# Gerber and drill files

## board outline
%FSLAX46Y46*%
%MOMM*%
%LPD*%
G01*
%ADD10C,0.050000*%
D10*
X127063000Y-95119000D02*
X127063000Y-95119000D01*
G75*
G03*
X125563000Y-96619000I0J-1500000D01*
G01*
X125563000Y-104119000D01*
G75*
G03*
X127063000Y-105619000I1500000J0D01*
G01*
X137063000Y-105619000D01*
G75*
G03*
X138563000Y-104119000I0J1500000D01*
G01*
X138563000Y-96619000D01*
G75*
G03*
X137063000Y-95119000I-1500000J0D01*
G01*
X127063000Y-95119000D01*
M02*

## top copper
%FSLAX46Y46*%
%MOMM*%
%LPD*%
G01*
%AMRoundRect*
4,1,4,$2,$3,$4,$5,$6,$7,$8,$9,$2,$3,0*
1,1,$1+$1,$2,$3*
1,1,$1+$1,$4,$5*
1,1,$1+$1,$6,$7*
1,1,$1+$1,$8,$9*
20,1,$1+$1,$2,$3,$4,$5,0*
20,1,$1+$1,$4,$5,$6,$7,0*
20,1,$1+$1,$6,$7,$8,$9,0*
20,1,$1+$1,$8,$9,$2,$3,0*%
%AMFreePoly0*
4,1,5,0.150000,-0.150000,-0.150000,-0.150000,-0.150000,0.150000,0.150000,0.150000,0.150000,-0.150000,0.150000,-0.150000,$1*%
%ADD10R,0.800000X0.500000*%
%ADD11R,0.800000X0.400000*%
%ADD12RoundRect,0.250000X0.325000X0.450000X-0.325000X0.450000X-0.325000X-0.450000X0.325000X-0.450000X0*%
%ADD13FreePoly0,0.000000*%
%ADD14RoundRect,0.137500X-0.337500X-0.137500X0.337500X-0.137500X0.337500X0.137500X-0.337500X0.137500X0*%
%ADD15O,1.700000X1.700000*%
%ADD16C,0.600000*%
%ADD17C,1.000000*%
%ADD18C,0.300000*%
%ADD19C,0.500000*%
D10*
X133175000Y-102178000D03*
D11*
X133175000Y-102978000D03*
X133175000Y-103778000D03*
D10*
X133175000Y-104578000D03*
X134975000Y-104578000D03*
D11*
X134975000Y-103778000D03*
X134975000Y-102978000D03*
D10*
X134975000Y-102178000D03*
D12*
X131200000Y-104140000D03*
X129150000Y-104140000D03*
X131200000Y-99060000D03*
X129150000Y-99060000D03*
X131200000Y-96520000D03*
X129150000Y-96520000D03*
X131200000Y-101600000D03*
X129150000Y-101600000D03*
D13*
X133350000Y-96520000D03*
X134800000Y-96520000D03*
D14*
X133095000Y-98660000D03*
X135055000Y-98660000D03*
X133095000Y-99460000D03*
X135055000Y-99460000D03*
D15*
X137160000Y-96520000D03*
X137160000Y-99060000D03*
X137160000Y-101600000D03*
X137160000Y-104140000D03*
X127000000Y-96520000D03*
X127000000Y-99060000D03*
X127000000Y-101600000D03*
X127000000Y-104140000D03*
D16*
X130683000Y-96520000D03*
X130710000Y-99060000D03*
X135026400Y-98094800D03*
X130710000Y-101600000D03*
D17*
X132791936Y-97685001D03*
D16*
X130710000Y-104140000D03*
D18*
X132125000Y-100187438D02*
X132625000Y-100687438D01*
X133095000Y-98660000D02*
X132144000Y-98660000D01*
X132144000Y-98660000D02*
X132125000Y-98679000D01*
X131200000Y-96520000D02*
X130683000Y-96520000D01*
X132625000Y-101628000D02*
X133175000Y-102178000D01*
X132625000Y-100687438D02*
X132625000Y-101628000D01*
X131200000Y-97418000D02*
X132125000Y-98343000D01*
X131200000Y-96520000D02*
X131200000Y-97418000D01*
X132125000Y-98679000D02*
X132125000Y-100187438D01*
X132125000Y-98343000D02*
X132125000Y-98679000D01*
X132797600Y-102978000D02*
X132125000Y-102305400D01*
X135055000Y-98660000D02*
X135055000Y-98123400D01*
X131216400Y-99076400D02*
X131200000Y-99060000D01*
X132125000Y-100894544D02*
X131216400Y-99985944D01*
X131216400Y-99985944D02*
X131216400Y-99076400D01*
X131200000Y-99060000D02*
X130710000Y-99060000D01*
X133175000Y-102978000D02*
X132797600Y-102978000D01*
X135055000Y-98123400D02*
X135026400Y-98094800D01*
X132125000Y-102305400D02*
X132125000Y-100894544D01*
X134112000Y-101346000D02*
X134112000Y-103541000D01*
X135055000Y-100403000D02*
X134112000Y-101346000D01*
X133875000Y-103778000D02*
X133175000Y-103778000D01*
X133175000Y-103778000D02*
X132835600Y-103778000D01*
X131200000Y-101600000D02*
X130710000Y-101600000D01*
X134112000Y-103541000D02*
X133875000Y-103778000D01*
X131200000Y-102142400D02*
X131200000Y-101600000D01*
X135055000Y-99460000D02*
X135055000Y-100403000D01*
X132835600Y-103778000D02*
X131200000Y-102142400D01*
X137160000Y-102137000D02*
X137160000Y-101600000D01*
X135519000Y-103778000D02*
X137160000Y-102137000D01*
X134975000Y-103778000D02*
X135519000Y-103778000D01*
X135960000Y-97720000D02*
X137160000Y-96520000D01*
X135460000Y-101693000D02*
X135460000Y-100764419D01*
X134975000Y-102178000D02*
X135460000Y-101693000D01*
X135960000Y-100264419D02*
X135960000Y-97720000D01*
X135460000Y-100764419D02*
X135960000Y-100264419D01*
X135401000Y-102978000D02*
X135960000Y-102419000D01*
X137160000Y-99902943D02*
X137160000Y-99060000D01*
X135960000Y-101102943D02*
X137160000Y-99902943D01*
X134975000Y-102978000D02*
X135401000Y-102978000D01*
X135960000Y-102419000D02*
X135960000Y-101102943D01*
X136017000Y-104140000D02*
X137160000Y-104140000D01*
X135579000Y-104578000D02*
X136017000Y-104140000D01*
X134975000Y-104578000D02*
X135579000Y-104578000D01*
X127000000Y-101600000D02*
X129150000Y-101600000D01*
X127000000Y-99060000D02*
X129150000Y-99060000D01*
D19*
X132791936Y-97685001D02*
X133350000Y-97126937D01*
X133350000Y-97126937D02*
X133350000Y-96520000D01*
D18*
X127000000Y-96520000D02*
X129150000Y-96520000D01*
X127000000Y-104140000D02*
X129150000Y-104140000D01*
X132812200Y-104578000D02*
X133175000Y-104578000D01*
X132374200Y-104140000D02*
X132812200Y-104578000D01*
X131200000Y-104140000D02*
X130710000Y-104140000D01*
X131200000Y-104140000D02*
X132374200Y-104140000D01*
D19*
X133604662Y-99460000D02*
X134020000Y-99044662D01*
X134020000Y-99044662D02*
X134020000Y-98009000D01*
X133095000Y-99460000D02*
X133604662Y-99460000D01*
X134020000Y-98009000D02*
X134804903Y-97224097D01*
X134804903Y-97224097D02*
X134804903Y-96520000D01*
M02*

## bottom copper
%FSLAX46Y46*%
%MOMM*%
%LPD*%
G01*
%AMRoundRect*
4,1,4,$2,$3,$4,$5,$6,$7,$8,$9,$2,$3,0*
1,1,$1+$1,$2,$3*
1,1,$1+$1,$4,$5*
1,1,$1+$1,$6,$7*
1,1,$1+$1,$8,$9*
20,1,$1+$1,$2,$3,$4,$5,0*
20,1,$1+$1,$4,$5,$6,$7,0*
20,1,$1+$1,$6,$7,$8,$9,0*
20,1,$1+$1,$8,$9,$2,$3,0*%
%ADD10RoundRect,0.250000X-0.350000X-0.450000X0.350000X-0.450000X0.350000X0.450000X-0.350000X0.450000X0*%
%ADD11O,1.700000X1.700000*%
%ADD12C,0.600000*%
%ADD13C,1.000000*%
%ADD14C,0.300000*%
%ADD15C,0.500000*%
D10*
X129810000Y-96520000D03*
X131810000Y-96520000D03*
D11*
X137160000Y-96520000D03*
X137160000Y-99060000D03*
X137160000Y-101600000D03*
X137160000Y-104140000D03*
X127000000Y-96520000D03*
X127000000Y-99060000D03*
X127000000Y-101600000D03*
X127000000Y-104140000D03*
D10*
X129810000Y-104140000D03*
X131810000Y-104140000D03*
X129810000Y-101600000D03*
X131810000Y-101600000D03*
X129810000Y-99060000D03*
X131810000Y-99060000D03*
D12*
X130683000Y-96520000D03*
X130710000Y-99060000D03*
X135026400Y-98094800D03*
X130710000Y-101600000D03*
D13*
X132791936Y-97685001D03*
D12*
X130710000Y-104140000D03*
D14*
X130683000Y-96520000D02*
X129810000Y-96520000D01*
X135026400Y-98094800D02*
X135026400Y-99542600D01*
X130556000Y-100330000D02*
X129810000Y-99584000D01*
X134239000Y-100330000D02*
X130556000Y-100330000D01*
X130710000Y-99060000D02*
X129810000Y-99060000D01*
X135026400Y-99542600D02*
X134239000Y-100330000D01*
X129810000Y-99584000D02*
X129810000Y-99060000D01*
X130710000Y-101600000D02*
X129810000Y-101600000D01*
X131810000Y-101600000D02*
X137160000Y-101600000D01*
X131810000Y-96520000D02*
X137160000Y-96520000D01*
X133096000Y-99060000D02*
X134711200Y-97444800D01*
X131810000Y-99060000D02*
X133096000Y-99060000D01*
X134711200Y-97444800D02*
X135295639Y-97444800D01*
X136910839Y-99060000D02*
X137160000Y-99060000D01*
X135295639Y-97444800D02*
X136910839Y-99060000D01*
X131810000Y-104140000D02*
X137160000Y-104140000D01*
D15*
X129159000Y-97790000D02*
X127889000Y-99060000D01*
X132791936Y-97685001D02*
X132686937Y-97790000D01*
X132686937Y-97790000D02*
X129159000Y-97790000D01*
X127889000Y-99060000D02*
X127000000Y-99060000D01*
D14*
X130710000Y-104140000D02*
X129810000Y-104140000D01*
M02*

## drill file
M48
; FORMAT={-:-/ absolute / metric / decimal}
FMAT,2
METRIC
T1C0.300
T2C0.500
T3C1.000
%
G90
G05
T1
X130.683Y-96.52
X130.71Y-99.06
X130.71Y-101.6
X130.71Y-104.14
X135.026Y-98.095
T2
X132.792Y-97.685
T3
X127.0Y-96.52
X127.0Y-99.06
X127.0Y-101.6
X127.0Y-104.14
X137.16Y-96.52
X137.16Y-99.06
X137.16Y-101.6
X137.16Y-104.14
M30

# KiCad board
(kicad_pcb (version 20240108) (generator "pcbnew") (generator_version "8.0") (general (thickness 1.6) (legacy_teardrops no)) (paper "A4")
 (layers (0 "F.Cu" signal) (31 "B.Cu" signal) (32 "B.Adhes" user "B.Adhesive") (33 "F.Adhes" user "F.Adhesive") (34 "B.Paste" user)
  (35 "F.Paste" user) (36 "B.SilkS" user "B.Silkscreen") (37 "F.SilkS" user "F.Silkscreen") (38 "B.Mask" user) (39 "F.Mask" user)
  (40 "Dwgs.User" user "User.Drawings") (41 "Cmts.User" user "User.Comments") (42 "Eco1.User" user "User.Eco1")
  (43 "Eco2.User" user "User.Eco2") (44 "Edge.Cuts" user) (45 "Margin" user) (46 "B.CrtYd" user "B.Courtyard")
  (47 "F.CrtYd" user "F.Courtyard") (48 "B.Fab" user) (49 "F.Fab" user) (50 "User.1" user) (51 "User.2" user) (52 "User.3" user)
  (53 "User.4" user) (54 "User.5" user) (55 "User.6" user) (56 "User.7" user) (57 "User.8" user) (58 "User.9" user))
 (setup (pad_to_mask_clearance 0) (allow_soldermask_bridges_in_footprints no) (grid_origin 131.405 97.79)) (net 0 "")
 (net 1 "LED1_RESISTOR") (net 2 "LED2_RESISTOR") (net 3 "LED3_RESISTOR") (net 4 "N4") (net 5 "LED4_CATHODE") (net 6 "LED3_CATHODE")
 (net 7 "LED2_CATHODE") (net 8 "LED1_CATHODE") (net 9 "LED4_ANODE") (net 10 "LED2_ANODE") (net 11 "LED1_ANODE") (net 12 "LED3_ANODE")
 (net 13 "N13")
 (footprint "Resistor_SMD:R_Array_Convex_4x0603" (layer "F.Cu") (at 134.075 103.378)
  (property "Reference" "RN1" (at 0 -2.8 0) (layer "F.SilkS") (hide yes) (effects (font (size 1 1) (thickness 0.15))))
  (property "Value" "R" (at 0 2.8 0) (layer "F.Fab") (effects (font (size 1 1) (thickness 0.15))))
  (pad "1" smd rect (at -0.9 -1.2) (size 0.8 0.5) (layers "F.Cu" "F.Paste" "F.Mask") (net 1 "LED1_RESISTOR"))
  (pad "2" smd rect (at -0.9 -0.4) (size 0.8 0.4) (layers "F.Cu" "F.Paste" "F.Mask") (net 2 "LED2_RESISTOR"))
  (pad "3" smd rect (at -0.9 0.4) (size 0.8 0.4) (layers "F.Cu" "F.Paste" "F.Mask") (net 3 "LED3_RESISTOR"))
  (pad "4" smd rect (at -0.9 1.2) (size 0.8 0.5) (layers "F.Cu" "F.Paste" "F.Mask") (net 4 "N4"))
  (pad "5" smd rect (at 0.9 1.2) (size 0.8 0.5) (layers "F.Cu" "F.Paste" "F.Mask") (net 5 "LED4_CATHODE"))
  (pad "6" smd rect (at 0.9 0.4) (size 0.8 0.4) (layers "F.Cu" "F.Paste" "F.Mask") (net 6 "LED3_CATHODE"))
  (pad "7" smd rect (at 0.9 -0.4) (size 0.8 0.4) (layers "F.Cu" "F.Paste" "F.Mask") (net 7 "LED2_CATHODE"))
  (pad "8" smd rect (at 0.9 -1.2) (size 0.8 0.5) (layers "F.Cu" "F.Paste" "F.Mask") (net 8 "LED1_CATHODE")))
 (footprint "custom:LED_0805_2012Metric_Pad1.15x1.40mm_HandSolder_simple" (layer "F.Cu") (at 130.175 104.14 180)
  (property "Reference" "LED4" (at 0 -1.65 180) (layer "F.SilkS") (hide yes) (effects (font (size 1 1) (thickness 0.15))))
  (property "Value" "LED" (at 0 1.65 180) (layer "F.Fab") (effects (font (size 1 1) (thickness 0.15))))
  (pad "1" smd roundrect (at -1.025 0 180) (size 1.15 1.4) (layers "F.Cu" "F.Paste" "F.Mask") (roundrect_rratio 0.217391) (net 4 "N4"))
  (pad "2" smd roundrect (at 1.025 0 180) (size 1.15 1.4) (layers "F.Cu" "F.Paste" "F.Mask") (roundrect_rratio 0.217391)
   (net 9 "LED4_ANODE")))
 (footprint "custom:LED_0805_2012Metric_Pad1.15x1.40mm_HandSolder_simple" (layer "F.Cu") (at 130.175 99.06 180)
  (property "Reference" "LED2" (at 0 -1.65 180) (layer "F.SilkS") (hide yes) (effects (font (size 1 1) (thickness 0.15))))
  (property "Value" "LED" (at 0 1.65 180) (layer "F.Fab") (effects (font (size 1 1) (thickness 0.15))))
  (pad "1" smd roundrect (at -1.025 0 180) (size 1.15 1.4) (layers "F.Cu" "F.Paste" "F.Mask") (roundrect_rratio 0.217391)
   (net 2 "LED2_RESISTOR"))
  (pad "2" smd roundrect (at 1.025 0 180) (size 1.15 1.4) (layers "F.Cu" "F.Paste" "F.Mask") (roundrect_rratio 0.217391)
   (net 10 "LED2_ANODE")))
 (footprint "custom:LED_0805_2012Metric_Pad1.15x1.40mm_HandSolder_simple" (layer "F.Cu") (at 130.175 96.52 180)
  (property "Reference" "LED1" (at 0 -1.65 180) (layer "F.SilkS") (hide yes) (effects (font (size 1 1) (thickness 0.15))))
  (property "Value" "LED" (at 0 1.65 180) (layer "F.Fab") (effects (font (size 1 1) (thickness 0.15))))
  (pad "1" smd roundrect (at -1.025 0 180) (size 1.15 1.4) (layers "F.Cu" "F.Paste" "F.Mask") (roundrect_rratio 0.217391)
   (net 1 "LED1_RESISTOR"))
  (pad "2" smd roundrect (at 1.025 0 180) (size 1.15 1.4) (layers "F.Cu" "F.Paste" "F.Mask") (roundrect_rratio 0.217391)
   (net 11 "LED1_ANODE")))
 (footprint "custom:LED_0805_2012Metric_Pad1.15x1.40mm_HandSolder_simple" (layer "F.Cu") (at 130.175 101.6 180)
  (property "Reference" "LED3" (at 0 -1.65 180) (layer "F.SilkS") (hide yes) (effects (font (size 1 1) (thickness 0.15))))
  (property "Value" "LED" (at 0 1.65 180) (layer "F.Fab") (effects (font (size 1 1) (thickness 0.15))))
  (pad "1" smd roundrect (at -1.025 0 180) (size 1.15 1.4) (layers "F.Cu" "F.Paste" "F.Mask") (roundrect_rratio 0.217391)
   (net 3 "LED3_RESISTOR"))
  (pad "2" smd roundrect (at 1.025 0 180) (size 1.15 1.4) (layers "F.Cu" "F.Paste" "F.Mask") (roundrect_rratio 0.217391)
   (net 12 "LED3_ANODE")))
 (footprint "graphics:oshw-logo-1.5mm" (layer "F.Cu") (at 134.874 100.711)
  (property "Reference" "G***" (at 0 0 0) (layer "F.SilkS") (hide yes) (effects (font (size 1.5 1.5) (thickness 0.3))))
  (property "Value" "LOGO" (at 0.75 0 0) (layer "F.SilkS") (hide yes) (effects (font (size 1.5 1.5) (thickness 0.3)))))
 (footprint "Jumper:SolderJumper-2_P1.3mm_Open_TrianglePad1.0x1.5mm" (layer "F.Cu") (at 134.075 96.52)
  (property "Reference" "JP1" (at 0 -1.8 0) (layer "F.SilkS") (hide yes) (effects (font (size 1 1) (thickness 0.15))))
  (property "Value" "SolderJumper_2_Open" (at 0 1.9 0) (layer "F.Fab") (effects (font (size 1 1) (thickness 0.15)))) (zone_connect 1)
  (pad "1" smd custom (at -0.725 0) (size 0.3 0.3) (layers "F.Cu" "F.Mask") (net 10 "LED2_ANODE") (zone_connect 2) (thermal_bridge_angle 45)
   (options (clearance outline) (anchor rect)) (primitives))
  (pad "2" smd custom (at 0.725 0) (size 0.3 0.3) (layers "F.Cu" "F.Mask") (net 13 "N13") (zone_connect 2) (thermal_bridge_angle 45)
   (options (clearance outline) (anchor rect)) (primitives)))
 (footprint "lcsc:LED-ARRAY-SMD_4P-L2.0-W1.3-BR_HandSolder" (layer "F.Cu") (at 134.075 99.06 180)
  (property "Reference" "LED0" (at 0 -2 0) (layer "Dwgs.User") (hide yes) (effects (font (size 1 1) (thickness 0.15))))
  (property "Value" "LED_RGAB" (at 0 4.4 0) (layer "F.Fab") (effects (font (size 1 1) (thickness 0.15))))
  (pad "1" smd roundrect (at 0.98 0.4) (size 0.95 0.55) (layers "F.Cu" "F.Paste" "F.Mask") (roundrect_rratio 0.25) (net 1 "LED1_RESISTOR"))
  (pad "2" smd roundrect (at -0.98 0.4) (size 0.95 0.55) (layers "F.Cu" "F.Paste" "F.Mask") (roundrect_rratio 0.25) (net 2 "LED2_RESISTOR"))
  (pad "3" smd roundrect (at 0.98 -0.4) (size 0.95 0.55) (layers "F.Cu" "F.Paste" "F.Mask") (roundrect_rratio 0.25) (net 13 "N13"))
  (pad "4" smd roundrect (at -0.98 -0.4) (size 0.95 0.55) (layers "F.Cu" "F.Paste" "F.Mask") (roundrect_rratio 0.25) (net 3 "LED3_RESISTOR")))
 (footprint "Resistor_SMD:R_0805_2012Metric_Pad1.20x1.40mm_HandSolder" (layer "B.Cu") (at 130.81 96.52)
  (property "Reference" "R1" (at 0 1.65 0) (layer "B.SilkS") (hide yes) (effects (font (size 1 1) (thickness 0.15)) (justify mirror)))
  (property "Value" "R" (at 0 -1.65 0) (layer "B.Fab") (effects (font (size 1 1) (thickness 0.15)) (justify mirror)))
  (pad "1" smd roundrect (at -1 0) (size 1.2 1.4) (layers "B.Cu" "B.Paste" "B.Mask") (roundrect_rratio 0.208333) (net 1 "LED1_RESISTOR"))
  (pad "2" smd roundrect (at 1 0) (size 1.2 1.4) (layers "B.Cu" "B.Paste" "B.Mask") (roundrect_rratio 0.208333) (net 8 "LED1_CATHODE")))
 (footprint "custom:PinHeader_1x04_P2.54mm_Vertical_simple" (layer "B.Cu") (at 137.16 96.52 180)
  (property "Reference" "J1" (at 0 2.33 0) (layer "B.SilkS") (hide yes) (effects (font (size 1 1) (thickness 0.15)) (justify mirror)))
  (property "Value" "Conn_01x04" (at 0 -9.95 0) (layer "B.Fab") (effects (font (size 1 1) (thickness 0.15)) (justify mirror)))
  (pad "1" thru_hole oval (at 0 0 180) (size 1.7 1.7) (drill 1) (layers "*.Cu" "*.Mask") (remove_unused_layers no) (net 8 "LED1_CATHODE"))
  (pad "2" thru_hole oval (at 0 -2.54 180) (size 1.7 1.7) (drill 1) (layers "*.Cu" "*.Mask") (remove_unused_layers no)
   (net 7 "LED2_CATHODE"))
  (pad "3" thru_hole oval (at 0 -5.08 180) (size 1.7 1.7) (drill 1) (layers "*.Cu" "*.Mask") (remove_unused_layers no)
   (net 6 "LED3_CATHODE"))
  (pad "4" thru_hole oval (at 0 -7.62 180) (size 1.7 1.7) (drill 1) (layers "*.Cu" "*.Mask") (remove_unused_layers no)
   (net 5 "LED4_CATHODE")))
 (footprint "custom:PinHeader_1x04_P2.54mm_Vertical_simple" (layer "B.Cu") (at 127 96.52 180)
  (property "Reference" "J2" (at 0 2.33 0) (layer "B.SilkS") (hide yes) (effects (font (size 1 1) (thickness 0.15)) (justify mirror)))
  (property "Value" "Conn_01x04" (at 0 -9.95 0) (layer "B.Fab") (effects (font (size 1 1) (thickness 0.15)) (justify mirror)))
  (pad "1" thru_hole oval (at 0 0 180) (size 1.7 1.7) (drill 1) (layers "*.Cu" "*.Mask") (remove_unused_layers no) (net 11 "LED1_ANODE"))
  (pad "2" thru_hole oval (at 0 -2.54 180) (size 1.7 1.7) (drill 1) (layers "*.Cu" "*.Mask") (remove_unused_layers no) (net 10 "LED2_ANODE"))
  (pad "3" thru_hole oval (at 0 -5.08 180) (size 1.7 1.7) (drill 1) (layers "*.Cu" "*.Mask") (remove_unused_layers no) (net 12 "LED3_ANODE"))
  (pad "4" thru_hole oval (at 0 -7.62 180) (size 1.7 1.7) (drill 1) (layers "*.Cu" "*.Mask") (remove_unused_layers no) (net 9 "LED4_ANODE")))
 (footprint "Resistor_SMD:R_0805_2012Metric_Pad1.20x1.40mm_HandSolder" (layer "B.Cu") (at 130.81 104.14)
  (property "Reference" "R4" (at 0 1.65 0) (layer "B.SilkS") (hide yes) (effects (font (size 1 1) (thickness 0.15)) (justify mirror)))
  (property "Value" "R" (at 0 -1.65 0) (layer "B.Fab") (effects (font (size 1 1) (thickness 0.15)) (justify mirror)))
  (pad "1" smd roundrect (at -1 0) (size 1.2 1.4) (layers "B.Cu" "B.Paste" "B.Mask") (roundrect_rratio 0.208333) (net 4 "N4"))
  (pad "2" smd roundrect (at 1 0) (size 1.2 1.4) (layers "B.Cu" "B.Paste" "B.Mask") (roundrect_rratio 0.208333) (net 5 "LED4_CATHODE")))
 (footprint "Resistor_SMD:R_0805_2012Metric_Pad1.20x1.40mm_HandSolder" (layer "B.Cu") (at 130.81 101.6)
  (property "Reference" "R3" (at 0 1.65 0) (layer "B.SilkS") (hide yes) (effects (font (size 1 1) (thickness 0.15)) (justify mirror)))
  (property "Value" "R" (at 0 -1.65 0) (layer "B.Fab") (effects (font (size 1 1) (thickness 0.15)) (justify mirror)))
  (pad "1" smd roundrect (at -1 0) (size 1.2 1.4) (layers "B.Cu" "B.Paste" "B.Mask") (roundrect_rratio 0.208333) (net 3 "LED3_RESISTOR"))
  (pad "2" smd roundrect (at 1 0) (size 1.2 1.4) (layers "B.Cu" "B.Paste" "B.Mask") (roundrect_rratio 0.208333) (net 6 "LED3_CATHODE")))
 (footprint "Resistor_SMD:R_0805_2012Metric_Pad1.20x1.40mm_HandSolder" (layer "B.Cu") (at 130.81 99.06)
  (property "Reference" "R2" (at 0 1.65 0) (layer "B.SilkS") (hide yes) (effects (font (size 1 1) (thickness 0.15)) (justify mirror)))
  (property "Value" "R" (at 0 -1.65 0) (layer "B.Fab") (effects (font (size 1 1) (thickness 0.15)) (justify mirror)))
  (pad "1" smd roundrect (at -1 0) (size 1.2 1.4) (layers "B.Cu" "B.Paste" "B.Mask") (roundrect_rratio 0.208333) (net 2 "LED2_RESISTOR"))
  (pad "2" smd roundrect (at 1 0) (size 1.2 1.4) (layers "B.Cu" "B.Paste" "B.Mask") (roundrect_rratio 0.208333) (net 7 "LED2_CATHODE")))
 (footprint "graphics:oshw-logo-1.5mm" (layer "B.Cu") (at 133.55 98.75 90)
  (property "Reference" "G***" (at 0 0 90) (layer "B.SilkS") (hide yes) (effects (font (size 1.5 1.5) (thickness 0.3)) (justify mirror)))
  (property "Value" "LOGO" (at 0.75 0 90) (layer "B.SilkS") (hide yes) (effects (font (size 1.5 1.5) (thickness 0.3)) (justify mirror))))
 (gr_poly
  (pts
   (arc (start 127.063 95.119) (mid 126.00234 95.55834) (end 125.563 96.619))
   (arc (start 125.563 104.119) (mid 126.00234 105.17966) (end 127.063 105.619))
   (arc (start 137.063 105.619) (mid 138.12366 105.17966) (end 138.563 104.119))
   (arc (start 138.563 96.619) (mid 138.12366 95.55834) (end 137.063 95.119)))
  (stroke (width 0.05) (type solid)) (fill none) (layer "Edge.Cuts"))
 (segment (start 132.125 100.187438) (end 132.625 100.687438) (width 0.3) (layer "F.Cu") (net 1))
 (segment (start 133.095 98.66) (end 132.144 98.66) (width 0.3) (layer "F.Cu") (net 1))
 (segment (start 132.144 98.66) (end 132.125 98.679) (width 0.3) (layer "F.Cu") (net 1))
 (segment (start 131.2 96.52) (end 130.683 96.52) (width 0.3) (layer "F.Cu") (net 1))
 (segment (start 132.625 101.628) (end 133.175 102.178) (width 0.3) (layer "F.Cu") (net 1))
 (segment (start 132.625 100.687438) (end 132.625 101.628) (width 0.3) (layer "F.Cu") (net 1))
 (segment (start 131.2 97.418) (end 132.125 98.343) (width 0.3) (layer "F.Cu") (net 1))
 (segment (start 131.2 96.52) (end 131.2 97.418) (width 0.3) (layer "F.Cu") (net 1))
 (segment (start 132.125 98.679) (end 132.125 100.187438) (width 0.3) (layer "F.Cu") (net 1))
 (segment (start 132.125 98.343) (end 132.125 98.679) (width 0.3) (layer "F.Cu") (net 1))
 (via (at 130.683 96.52) (size 0.6) (drill 0.3) (layers "F.Cu" "B.Cu") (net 1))
 (segment (start 130.683 96.52) (end 129.81 96.52) (width 0.3) (layer "B.Cu") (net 1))
 (segment (start 132.7976 102.978) (end 132.125 102.3054) (width 0.3) (layer "F.Cu") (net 2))
 (segment (start 135.055 98.66) (end 135.055 98.1234) (width 0.3) (layer "F.Cu") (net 2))
 (segment (start 131.2164 99.0764) (end 131.2 99.06) (width 0.3) (layer "F.Cu") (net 2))
 (segment (start 132.125 100.894544) (end 131.2164 99.985944) (width 0.3) (layer "F.Cu") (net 2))
 (segment (start 131.2164 99.985944) (end 131.2164 99.0764) (width 0.3) (layer "F.Cu") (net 2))
 (segment (start 131.2 99.06) (end 130.71 99.06) (width 0.3) (layer "F.Cu") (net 2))
 (segment (start 133.175 102.978) (end 132.7976 102.978) (width 0.3) (layer "F.Cu") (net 2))
 (segment (start 135.055 98.1234) (end 135.0264 98.0948) (width 0.3) (layer "F.Cu") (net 2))
 (segment (start 132.125 102.3054) (end 132.125 100.894544) (width 0.3) (layer "F.Cu") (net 2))
 (via (at 130.71 99.06) (size 0.6) (drill 0.3) (layers "F.Cu" "B.Cu") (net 2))
 (via (at 135.0264 98.0948) (size 0.6) (drill 0.3) (layers "F.Cu" "B.Cu") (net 2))
 (segment (start 135.0264 98.0948) (end 135.0264 99.5426) (width 0.3) (layer "B.Cu") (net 2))
 (segment (start 130.556 100.33) (end 129.81 99.584) (width 0.3) (layer "B.Cu") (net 2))
 (segment (start 134.239 100.33) (end 130.556 100.33) (width 0.3) (layer "B.Cu") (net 2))
 (segment (start 130.71 99.06) (end 129.81 99.06) (width 0.3) (layer "B.Cu") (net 2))
 (segment (start 135.0264 99.5426) (end 134.239 100.33) (width 0.3) (layer "B.Cu") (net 2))
 (segment (start 129.81 99.584) (end 129.81 99.06) (width 0.3) (layer "B.Cu") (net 2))
 (segment (start 134.112 101.346) (end 134.112 103.541) (width 0.3) (layer "F.Cu") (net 3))
 (segment (start 135.055 100.403) (end 134.112 101.346) (width 0.3) (layer "F.Cu") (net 3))
 (segment (start 133.875 103.778) (end 133.175 103.778) (width 0.3) (layer "F.Cu") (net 3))
 (segment (start 133.175 103.778) (end 132.8356 103.778) (width 0.3) (layer "F.Cu") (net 3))
 (segment (start 131.2 101.6) (end 130.71 101.6) (width 0.3) (layer "F.Cu") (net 3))
 (segment (start 134.112 103.541) (end 133.875 103.778) (width 0.3) (layer "F.Cu") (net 3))
 (segment (start 131.2 102.1424) (end 131.2 101.6) (width 0.3) (layer "F.Cu") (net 3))
 (segment (start 135.055 99.46) (end 135.055 100.403) (width 0.3) (layer "F.Cu") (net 3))
 (segment (start 132.8356 103.778) (end 131.2 102.1424) (width 0.3) (layer "F.Cu") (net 3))
 (via (at 130.71 101.6) (size 0.6) (drill 0.3) (layers "F.Cu" "B.Cu") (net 3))
 (segment (start 130.71 101.6) (end 129.81 101.6) (width 0.3) (layer "B.Cu") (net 3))
 (segment (start 137.16 102.137) (end 137.16 101.6) (width 0.3) (layer "F.Cu") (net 6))
 (segment (start 135.519 103.778) (end 137.16 102.137) (width 0.3) (layer "F.Cu") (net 6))
 (segment (start 134.975 103.778) (end 135.519 103.778) (width 0.3) (layer "F.Cu") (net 6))
 (segment (start 131.81 101.6) (end 137.16 101.6) (width 0.3) (layer "B.Cu") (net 6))
 (segment (start 135.96 97.72) (end 137.16 96.52) (width 0.3) (layer "F.Cu") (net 8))
 (segment (start 135.46 101.693) (end 135.46 100.764419) (width 0.3) (layer "F.Cu") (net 8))
 (segment (start 134.975 102.178) (end 135.46 101.693) (width 0.3) (layer "F.Cu") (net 8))
 (segment (start 135.96 100.264419) (end 135.96 97.72) (width 0.3) (layer "F.Cu") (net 8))
 (segment (start 135.46 100.764419) (end 135.96 100.264419) (width 0.3) (layer "F.Cu") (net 8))
 (segment (start 131.81 96.52) (end 137.16 96.52) (width 0.3) (layer "B.Cu") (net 8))
 (segment (start 135.401 102.978) (end 135.96 102.419) (width 0.3) (layer "F.Cu") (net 7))
 (segment (start 137.16 99.902943) (end 137.16 99.06) (width 0.3) (layer "F.Cu") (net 7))
 (segment (start 135.96 101.102943) (end 137.16 99.902943) (width 0.3) (layer "F.Cu") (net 7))
 (segment (start 134.975 102.978) (end 135.401 102.978) (width 0.3) (layer "F.Cu") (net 7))
 (segment (start 135.96 102.419) (end 135.96 101.102943) (width 0.3) (layer "F.Cu") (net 7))
 (segment (start 133.096 99.06) (end 134.7112 97.4448) (width 0.3) (layer "B.Cu") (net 7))
 (segment (start 131.81 99.06) (end 133.096 99.06) (width 0.3) (layer "B.Cu") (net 7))
 (segment (start 134.7112 97.4448) (end 135.295639 97.4448) (width 0.3) (layer "B.Cu") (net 7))
 (segment (start 136.910839 99.06) (end 137.16 99.06) (width 0.3) (layer "B.Cu") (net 7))
 (segment (start 135.295639 97.4448) (end 136.910839 99.06) (width 0.3) (layer "B.Cu") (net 7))
 (segment (start 136.017 104.14) (end 137.16 104.14) (width 0.3) (layer "F.Cu") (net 5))
 (segment (start 135.579 104.578) (end 136.017 104.14) (width 0.3) (layer "F.Cu") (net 5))
 (segment (start 134.975 104.578) (end 135.579 104.578) (width 0.3) (layer "F.Cu") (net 5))
 (segment (start 131.81 104.14) (end 137.16 104.14) (width 0.3) (layer "B.Cu") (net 5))
 (segment (start 127 101.6) (end 129.15 101.6) (width 0.3) (layer "F.Cu") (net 12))
 (segment (start 127 99.06) (end 129.15 99.06) (width 0.3) (layer "F.Cu") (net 10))
 (segment (start 132.791936 97.685001) (end 133.35 97.126937) (width 0.5) (layer "F.Cu") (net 10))
 (segment (start 133.35 97.126937) (end 133.35 96.52) (width 0.5) (layer "F.Cu") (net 10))
 (via (at 132.791936 97.685001) (size 1) (drill 0.5) (layers "F.Cu" "B.Cu") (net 10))
 (segment (start 129.159 97.79) (end 127.889 99.06) (width 0.5) (layer "B.Cu") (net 10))
 (segment (start 132.791936 97.685001) (end 132.686937 97.79) (width 0.5) (layer "B.Cu") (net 10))
 (segment (start 132.686937 97.79) (end 129.159 97.79) (width 0.5) (layer "B.Cu") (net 10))
 (segment (start 127.889 99.06) (end 127 99.06) (width 0.5) (layer "B.Cu") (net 10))
 (segment (start 127 96.52) (end 129.15 96.52) (width 0.3) (layer "F.Cu") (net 11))
 (segment (start 127 104.14) (end 129.15 104.14) (width 0.3) (layer "F.Cu") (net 9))
 (segment (start 132.8122 104.578) (end 133.175 104.578) (width 0.3) (layer "F.Cu") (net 4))
 (segment (start 132.3742 104.14) (end 132.8122 104.578) (width 0.3) (layer "F.Cu") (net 4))
 (segment (start 131.2 104.14) (end 130.71 104.14) (width 0.3) (layer "F.Cu") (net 4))
 (segment (start 131.2 104.14) (end 132.3742 104.14) (width 0.3) (layer "F.Cu") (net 4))
 (via (at 130.71 104.14) (size 0.6) (drill 0.3) (layers "F.Cu" "B.Cu") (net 4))
 (segment (start 130.71 104.14) (end 129.81 104.14) (width 0.3) (layer "B.Cu") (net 4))
 (segment (start 133.604662 99.46) (end 134.02 99.044662) (width 0.5) (layer "F.Cu") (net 13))
 (segment (start 134.02 99.044662) (end 134.02 98.009) (width 0.5) (layer "F.Cu") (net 13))
 (segment (start 133.095 99.46) (end 133.604662 99.46) (width 0.5) (layer "F.Cu") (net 13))
 (segment (start 134.02 98.009) (end 134.804903 97.224097) (width 0.5) (layer "F.Cu") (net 13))
 (segment (start 134.804903 97.224097) (end 134.804903 96.52) (width 0.5) (layer "F.Cu") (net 13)))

